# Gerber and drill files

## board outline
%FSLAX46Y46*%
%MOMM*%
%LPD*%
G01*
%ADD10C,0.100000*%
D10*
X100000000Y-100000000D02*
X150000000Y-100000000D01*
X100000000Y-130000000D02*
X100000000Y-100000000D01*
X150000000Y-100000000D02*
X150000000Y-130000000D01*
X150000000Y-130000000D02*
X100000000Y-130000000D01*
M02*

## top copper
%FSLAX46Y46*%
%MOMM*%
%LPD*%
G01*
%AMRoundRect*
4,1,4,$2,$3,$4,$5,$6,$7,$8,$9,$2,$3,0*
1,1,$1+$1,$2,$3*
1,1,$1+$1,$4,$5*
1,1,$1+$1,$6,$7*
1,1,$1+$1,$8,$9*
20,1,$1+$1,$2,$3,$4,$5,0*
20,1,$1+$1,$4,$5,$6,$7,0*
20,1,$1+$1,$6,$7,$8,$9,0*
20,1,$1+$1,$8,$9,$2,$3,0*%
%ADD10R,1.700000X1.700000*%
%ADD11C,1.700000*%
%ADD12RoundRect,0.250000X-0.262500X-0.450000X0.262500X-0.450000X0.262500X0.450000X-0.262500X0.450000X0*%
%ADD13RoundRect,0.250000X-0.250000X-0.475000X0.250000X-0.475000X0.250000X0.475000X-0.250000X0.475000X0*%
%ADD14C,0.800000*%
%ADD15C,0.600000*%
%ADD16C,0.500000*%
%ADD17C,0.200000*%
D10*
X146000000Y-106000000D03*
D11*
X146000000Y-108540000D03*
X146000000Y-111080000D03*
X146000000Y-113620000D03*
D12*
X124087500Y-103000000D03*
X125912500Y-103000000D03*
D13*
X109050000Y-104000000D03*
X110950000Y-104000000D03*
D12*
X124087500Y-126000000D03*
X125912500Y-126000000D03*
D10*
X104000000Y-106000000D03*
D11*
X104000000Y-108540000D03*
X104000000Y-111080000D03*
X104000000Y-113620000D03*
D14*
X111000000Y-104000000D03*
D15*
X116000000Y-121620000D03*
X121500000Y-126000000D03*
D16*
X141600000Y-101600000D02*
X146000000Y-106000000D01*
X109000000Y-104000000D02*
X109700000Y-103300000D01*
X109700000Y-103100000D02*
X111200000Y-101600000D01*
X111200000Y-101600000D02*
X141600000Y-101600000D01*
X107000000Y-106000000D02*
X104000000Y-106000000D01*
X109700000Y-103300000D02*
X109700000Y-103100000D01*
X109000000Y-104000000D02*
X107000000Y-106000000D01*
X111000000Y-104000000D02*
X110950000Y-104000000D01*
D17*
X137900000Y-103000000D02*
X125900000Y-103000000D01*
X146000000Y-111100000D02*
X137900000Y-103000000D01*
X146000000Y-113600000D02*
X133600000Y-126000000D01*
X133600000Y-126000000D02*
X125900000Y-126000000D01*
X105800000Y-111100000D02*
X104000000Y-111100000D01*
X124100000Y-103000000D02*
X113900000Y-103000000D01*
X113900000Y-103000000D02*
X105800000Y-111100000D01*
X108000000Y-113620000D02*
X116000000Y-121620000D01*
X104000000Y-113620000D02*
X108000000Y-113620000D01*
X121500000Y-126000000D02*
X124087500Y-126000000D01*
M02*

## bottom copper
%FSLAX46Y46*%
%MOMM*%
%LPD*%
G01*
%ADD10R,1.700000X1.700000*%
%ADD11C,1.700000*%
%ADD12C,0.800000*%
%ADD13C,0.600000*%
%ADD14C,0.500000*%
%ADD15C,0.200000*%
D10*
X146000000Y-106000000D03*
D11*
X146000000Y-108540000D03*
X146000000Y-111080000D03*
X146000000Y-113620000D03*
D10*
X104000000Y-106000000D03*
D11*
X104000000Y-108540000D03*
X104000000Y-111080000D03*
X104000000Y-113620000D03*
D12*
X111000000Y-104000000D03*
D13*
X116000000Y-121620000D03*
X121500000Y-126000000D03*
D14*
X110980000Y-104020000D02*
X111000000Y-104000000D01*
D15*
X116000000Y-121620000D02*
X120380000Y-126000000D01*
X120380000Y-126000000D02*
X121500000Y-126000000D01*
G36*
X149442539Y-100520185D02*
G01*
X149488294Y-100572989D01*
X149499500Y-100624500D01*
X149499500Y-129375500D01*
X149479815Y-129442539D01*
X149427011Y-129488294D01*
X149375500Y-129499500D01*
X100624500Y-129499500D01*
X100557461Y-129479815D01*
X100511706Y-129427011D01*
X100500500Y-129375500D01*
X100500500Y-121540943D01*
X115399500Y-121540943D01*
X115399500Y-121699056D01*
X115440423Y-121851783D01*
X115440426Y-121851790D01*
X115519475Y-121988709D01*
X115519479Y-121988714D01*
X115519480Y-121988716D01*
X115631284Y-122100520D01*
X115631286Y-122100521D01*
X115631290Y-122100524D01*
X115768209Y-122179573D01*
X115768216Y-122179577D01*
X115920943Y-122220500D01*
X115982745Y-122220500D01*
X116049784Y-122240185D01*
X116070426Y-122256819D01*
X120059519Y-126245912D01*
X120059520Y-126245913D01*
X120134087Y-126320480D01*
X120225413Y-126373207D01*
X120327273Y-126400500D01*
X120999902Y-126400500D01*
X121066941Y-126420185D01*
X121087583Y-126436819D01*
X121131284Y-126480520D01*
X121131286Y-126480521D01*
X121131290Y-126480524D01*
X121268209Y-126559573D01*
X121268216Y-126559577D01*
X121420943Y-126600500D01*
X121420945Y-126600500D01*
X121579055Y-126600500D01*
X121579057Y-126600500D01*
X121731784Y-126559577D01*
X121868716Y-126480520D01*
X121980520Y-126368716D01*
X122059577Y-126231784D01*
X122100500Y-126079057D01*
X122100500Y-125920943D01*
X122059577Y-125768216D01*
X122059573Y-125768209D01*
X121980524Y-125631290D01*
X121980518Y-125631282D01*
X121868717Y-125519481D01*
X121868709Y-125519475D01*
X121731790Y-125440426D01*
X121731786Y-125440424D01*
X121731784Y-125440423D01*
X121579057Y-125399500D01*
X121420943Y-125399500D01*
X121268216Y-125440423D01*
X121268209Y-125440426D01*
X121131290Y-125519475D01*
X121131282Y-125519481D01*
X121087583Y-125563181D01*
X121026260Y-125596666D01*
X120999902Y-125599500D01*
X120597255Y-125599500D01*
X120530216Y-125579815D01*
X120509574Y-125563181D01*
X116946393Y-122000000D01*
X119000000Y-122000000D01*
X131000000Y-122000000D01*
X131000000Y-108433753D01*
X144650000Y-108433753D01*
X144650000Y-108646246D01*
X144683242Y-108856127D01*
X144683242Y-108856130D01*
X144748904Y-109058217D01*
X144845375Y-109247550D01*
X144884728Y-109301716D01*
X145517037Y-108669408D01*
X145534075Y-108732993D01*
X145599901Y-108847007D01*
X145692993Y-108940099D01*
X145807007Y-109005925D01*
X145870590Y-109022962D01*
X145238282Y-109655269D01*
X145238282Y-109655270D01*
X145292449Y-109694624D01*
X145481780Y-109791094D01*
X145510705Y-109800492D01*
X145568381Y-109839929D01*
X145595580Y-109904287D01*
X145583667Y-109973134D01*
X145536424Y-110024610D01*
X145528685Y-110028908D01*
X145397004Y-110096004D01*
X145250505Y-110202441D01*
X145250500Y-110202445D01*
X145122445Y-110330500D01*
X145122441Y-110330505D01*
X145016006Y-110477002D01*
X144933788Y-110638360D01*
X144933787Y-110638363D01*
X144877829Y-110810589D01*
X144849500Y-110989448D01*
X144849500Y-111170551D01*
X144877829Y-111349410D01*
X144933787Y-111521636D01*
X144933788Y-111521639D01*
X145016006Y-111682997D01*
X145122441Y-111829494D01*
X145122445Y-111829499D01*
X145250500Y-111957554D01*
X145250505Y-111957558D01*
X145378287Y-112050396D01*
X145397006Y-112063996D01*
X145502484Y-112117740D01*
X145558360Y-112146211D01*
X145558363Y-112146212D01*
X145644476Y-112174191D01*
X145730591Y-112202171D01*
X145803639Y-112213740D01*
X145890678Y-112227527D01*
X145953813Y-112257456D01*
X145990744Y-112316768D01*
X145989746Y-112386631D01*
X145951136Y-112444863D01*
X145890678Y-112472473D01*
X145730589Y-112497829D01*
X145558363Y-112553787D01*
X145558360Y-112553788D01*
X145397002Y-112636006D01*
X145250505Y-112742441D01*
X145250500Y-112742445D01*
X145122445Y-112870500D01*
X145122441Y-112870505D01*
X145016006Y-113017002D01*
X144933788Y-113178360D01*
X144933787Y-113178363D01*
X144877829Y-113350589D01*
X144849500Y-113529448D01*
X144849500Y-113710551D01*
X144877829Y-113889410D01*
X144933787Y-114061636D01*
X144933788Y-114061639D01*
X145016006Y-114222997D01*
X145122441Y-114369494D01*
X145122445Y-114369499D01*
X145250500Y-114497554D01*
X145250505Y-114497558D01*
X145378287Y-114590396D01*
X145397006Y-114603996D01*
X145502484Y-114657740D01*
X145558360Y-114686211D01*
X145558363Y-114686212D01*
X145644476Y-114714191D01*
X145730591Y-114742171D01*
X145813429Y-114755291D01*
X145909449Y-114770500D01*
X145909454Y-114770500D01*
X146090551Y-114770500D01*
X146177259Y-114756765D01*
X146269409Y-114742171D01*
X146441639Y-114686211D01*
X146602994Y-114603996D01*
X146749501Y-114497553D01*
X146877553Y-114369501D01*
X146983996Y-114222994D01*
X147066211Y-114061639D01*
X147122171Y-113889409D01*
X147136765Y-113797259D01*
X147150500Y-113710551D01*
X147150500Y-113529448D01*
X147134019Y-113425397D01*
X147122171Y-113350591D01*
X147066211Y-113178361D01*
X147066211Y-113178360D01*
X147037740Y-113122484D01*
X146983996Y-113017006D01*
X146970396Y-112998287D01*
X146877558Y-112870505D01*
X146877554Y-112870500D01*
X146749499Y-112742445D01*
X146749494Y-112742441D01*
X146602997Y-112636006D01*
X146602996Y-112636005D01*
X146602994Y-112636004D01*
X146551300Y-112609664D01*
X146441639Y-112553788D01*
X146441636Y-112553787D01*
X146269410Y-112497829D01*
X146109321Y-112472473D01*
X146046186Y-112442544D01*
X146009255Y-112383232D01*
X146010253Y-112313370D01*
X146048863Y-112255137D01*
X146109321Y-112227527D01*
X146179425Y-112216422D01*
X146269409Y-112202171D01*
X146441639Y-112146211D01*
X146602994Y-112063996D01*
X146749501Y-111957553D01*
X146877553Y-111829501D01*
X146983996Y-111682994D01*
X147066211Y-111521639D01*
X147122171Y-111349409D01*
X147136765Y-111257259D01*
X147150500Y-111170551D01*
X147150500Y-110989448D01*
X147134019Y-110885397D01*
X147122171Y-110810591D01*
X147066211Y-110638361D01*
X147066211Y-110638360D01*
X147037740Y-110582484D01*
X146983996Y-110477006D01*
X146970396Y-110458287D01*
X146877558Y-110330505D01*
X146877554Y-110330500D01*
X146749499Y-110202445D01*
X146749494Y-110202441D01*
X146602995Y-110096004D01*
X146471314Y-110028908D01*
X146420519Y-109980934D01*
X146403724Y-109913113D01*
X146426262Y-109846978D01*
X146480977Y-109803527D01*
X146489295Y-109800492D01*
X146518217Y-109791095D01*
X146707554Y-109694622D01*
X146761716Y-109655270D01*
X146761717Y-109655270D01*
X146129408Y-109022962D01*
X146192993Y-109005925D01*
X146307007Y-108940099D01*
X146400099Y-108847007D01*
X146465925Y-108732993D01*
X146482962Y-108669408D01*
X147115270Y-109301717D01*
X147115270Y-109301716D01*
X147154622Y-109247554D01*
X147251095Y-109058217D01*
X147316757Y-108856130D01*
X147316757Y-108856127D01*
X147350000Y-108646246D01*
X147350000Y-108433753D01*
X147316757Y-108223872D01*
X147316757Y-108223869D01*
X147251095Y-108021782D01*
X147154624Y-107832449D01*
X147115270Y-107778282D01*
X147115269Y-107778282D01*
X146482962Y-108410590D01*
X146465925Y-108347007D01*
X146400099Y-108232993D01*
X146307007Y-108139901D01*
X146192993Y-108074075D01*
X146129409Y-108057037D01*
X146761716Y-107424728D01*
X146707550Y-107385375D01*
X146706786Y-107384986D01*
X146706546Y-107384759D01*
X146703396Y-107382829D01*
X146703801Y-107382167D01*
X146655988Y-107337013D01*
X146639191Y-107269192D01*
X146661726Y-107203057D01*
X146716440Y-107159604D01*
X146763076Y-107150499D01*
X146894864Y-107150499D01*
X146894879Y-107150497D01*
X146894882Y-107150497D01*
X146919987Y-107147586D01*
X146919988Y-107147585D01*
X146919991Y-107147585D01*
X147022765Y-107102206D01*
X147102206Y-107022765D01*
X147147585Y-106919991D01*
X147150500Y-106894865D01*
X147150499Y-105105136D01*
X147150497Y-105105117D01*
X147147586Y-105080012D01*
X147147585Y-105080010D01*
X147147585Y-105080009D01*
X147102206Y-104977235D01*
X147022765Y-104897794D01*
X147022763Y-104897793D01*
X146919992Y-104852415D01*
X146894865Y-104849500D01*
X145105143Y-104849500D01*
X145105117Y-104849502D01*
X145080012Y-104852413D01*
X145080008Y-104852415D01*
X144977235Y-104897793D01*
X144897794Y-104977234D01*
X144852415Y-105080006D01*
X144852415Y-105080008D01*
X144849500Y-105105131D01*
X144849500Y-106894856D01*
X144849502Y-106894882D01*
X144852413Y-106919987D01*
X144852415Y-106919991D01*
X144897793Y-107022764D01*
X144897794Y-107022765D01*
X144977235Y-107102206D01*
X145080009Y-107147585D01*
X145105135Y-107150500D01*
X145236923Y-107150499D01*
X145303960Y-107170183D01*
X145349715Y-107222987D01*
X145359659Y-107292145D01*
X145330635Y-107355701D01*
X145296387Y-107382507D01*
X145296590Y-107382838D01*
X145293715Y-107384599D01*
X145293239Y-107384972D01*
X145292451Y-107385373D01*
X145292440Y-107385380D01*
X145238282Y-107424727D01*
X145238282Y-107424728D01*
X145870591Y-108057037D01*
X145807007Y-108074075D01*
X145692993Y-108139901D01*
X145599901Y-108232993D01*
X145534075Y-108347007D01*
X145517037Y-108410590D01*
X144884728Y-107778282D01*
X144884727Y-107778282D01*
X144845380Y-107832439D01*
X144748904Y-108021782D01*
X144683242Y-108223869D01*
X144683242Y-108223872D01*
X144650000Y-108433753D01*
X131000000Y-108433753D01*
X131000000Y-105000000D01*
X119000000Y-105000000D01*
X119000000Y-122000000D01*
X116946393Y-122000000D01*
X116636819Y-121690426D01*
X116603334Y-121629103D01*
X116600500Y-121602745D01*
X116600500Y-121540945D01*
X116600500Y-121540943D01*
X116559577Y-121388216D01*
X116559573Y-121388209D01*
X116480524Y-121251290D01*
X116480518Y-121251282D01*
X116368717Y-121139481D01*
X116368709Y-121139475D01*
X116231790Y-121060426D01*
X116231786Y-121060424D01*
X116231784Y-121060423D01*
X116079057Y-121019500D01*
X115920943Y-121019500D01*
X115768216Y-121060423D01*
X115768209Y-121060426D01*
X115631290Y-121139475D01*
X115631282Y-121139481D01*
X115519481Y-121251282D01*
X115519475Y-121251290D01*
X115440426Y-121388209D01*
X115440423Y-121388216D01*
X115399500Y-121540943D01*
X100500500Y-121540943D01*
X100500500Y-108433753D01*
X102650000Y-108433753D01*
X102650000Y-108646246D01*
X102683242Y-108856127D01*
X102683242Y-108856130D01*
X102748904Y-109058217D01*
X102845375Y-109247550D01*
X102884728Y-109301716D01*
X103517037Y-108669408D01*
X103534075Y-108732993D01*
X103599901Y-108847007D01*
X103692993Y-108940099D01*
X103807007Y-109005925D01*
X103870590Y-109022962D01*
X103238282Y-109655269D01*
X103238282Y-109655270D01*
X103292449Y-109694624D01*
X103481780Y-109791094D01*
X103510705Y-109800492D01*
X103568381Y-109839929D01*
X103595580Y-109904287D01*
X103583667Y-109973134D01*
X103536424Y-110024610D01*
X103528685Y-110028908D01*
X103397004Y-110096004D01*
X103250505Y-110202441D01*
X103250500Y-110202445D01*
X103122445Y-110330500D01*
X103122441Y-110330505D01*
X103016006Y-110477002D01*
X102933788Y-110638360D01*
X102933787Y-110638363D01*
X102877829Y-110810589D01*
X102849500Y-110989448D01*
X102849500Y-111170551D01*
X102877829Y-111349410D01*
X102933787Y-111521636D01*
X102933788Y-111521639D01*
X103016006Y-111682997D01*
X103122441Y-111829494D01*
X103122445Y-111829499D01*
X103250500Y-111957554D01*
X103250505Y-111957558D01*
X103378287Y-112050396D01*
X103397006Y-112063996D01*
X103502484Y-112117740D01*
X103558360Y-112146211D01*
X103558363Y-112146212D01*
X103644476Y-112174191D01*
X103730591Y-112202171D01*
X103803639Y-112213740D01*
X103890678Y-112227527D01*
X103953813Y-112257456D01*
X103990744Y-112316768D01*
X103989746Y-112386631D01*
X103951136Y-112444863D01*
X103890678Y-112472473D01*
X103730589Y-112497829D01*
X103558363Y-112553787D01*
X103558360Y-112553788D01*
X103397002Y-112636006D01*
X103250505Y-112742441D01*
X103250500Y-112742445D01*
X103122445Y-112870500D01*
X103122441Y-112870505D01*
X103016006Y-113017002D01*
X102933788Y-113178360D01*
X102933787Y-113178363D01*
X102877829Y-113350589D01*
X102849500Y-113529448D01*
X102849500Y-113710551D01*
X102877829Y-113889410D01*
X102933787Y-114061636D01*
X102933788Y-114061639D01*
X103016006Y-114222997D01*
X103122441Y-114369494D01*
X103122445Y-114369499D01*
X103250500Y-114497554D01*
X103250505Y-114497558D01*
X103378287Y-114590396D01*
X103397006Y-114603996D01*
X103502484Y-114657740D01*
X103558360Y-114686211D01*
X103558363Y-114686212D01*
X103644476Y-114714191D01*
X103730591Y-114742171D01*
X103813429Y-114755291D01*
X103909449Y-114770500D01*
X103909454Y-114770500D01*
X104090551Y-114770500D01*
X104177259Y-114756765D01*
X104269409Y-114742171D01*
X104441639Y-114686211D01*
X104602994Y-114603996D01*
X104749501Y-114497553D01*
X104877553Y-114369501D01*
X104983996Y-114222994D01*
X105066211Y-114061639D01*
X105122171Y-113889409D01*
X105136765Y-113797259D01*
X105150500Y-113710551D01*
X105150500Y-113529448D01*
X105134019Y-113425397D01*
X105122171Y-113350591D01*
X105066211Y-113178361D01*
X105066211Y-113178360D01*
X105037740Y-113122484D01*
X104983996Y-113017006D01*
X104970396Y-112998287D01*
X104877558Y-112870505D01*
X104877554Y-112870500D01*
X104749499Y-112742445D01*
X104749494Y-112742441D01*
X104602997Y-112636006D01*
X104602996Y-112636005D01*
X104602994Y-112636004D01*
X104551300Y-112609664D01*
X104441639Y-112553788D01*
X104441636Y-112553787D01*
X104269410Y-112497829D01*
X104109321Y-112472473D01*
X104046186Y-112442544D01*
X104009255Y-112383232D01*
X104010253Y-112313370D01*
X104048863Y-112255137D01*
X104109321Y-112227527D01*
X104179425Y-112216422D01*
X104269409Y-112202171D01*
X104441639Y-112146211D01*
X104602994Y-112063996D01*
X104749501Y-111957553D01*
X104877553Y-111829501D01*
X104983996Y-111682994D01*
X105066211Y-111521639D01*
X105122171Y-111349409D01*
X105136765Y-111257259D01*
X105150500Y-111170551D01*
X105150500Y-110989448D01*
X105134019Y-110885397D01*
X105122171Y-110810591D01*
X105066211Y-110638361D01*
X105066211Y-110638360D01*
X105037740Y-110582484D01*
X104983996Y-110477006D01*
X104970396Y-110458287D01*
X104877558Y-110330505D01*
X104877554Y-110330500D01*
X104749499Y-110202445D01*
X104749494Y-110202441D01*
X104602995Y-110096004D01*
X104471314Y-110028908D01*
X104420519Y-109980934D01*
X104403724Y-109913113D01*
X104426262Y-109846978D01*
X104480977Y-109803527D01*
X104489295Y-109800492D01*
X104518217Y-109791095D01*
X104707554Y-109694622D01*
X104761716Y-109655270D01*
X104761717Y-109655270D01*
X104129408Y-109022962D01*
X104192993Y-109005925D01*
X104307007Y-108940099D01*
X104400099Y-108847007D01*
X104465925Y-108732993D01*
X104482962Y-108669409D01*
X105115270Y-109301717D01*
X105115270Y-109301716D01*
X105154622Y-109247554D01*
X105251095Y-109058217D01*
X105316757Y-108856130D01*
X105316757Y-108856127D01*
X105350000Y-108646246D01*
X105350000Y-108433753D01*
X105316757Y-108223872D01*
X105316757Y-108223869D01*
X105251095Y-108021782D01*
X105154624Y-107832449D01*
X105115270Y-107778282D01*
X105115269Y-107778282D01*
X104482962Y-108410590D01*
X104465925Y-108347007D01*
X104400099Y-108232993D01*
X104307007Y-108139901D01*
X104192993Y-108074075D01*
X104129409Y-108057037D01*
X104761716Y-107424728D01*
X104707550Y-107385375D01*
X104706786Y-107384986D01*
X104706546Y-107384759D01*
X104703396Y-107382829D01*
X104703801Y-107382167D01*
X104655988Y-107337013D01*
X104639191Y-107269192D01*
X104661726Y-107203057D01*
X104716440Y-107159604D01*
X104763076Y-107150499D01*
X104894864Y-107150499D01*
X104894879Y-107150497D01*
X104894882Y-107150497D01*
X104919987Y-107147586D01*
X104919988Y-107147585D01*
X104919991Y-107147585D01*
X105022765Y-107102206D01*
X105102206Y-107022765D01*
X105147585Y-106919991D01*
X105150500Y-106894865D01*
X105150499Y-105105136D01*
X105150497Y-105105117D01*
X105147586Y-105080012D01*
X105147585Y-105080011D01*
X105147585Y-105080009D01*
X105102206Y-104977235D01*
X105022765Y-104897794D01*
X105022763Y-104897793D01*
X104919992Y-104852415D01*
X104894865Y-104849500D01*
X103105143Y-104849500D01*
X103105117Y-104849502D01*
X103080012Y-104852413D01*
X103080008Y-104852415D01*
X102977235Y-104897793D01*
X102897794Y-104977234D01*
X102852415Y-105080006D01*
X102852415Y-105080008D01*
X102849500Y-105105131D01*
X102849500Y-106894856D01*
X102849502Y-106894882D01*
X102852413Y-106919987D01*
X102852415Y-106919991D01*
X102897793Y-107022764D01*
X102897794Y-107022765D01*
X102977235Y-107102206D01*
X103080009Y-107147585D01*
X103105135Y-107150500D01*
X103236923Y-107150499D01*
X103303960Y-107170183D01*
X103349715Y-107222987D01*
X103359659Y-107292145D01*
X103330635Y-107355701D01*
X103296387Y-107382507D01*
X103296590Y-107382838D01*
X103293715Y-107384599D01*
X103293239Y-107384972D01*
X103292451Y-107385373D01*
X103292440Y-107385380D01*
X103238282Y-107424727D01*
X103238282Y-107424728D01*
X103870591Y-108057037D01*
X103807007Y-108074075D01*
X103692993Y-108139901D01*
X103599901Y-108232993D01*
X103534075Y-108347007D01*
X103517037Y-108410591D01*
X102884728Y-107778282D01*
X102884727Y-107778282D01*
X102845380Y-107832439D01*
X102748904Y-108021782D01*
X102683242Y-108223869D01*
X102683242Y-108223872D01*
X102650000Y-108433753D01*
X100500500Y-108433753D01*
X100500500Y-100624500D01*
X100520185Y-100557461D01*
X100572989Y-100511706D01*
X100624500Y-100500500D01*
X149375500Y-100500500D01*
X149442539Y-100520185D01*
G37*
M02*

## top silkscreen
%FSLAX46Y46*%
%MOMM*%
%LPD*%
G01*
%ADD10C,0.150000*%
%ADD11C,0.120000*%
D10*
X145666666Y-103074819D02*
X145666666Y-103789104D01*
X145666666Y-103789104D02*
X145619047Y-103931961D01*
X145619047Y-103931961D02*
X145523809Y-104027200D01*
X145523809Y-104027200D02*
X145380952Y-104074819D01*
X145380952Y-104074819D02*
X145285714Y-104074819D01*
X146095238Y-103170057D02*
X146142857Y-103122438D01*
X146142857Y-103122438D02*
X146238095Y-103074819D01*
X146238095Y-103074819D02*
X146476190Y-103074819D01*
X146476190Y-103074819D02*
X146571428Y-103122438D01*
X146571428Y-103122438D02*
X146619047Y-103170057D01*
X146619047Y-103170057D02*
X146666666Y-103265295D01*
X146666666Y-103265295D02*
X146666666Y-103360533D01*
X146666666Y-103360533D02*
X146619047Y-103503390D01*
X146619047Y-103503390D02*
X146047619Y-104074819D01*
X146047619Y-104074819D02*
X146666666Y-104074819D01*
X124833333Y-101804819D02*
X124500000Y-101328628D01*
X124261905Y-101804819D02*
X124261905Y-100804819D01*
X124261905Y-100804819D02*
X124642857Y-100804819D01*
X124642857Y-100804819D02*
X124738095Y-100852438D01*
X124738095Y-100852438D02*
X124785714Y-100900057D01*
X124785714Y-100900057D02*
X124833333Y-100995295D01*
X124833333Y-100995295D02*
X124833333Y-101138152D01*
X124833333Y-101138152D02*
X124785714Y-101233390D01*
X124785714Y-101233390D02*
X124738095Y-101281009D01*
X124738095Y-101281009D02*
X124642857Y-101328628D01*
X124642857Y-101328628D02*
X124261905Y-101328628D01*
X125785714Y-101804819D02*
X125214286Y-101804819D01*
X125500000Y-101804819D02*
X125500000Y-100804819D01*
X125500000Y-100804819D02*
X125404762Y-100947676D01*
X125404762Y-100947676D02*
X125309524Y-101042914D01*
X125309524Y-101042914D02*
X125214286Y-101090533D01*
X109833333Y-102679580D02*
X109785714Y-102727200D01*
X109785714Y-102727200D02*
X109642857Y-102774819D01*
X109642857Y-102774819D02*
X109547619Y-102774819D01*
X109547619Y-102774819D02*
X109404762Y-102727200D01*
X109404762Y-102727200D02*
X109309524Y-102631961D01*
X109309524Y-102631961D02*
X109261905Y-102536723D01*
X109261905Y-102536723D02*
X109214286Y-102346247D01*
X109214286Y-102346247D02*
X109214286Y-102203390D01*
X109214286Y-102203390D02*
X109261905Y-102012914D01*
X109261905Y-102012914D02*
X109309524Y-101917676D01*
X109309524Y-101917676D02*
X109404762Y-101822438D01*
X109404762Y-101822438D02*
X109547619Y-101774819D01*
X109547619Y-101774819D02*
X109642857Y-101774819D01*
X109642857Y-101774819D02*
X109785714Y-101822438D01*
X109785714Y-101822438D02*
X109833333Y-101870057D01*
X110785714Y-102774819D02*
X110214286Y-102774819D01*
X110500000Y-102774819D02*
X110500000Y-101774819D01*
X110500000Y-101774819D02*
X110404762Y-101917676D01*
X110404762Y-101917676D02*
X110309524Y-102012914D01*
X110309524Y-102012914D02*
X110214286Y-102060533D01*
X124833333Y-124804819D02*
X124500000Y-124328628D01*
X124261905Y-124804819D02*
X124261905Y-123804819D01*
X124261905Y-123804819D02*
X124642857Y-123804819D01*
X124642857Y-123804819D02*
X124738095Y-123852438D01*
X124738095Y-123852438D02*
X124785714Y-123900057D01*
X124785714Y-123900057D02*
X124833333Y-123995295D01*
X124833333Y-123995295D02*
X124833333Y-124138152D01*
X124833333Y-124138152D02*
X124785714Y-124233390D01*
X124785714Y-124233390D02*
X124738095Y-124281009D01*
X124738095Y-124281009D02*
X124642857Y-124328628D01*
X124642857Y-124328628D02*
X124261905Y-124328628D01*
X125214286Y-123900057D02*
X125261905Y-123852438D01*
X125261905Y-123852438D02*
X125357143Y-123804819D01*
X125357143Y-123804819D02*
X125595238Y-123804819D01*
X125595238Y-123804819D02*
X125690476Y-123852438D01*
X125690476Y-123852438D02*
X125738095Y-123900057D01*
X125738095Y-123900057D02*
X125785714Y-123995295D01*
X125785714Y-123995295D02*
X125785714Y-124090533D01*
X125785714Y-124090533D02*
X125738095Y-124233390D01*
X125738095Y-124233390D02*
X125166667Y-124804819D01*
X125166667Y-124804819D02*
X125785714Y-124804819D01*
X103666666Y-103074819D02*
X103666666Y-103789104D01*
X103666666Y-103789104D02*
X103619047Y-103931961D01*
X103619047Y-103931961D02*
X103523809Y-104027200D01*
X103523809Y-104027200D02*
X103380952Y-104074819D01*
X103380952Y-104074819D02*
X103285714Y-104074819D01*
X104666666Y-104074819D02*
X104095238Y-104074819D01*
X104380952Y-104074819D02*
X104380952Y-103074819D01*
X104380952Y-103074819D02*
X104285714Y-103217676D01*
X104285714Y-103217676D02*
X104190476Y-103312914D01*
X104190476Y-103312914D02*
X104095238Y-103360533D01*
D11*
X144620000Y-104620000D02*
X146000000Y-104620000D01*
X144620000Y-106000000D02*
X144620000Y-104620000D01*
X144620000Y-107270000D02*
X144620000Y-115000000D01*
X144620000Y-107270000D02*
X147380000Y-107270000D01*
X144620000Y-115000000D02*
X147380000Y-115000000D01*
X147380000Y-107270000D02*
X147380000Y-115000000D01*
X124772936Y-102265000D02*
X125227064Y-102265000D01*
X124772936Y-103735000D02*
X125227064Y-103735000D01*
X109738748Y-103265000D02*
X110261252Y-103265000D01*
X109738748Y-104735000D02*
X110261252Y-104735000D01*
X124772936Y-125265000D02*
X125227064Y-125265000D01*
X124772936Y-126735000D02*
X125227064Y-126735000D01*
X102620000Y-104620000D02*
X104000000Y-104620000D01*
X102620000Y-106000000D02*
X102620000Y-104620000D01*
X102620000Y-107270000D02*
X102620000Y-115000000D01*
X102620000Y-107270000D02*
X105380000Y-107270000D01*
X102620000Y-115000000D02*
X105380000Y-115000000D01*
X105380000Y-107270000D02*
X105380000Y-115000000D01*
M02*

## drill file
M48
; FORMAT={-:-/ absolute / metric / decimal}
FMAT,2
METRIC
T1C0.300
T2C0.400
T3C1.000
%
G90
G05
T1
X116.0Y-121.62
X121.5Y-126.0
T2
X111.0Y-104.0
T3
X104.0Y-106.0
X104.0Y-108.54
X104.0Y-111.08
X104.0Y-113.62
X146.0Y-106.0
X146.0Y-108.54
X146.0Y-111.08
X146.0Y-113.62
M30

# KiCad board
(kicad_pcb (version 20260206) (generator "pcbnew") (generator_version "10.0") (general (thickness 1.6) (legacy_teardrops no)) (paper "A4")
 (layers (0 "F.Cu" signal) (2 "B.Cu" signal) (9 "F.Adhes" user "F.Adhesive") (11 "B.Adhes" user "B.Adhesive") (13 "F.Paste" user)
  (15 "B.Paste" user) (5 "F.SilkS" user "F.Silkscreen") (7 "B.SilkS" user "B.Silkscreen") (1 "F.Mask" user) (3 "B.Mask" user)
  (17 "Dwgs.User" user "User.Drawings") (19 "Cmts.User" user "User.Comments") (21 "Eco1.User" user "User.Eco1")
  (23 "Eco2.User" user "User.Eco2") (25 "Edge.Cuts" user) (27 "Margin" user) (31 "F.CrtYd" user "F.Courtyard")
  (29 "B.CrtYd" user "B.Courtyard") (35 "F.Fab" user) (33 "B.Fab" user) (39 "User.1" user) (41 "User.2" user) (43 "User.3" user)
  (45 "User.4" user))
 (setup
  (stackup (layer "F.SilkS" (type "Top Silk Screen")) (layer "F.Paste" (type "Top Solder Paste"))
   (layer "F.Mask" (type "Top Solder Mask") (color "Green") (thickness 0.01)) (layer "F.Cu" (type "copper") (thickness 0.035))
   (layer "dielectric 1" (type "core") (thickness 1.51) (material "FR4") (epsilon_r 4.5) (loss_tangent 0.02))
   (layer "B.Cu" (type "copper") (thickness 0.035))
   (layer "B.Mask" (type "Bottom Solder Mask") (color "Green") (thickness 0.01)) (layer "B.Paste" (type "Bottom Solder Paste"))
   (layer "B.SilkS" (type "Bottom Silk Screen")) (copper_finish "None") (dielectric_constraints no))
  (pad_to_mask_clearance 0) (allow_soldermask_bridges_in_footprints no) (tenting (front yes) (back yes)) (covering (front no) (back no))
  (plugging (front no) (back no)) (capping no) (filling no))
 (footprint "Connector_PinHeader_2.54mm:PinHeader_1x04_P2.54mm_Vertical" (layer "F.Cu") (at 146 106)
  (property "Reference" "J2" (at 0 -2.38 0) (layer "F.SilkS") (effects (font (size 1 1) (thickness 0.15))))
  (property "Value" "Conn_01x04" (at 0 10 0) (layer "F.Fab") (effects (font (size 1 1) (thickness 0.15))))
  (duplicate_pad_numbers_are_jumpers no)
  (fp_line (start -1.38 -1.38) (end 0 -1.38) (stroke (width 0.12) (type solid)) (layer "F.SilkS"))
  (fp_line (start -1.38 0) (end -1.38 -1.38) (stroke (width 0.12) (type solid)) (layer "F.SilkS"))
  (fp_line (start -1.38 1.27) (end -1.38 9) (stroke (width 0.12) (type solid)) (layer "F.SilkS"))
  (fp_line (start -1.38 1.27) (end 1.38 1.27) (stroke (width 0.12) (type solid)) (layer "F.SilkS"))
  (fp_line (start -1.38 9) (end 1.38 9) (stroke (width 0.12) (type solid)) (layer "F.SilkS"))
  (fp_line (start 1.38 1.27) (end 1.38 9) (stroke (width 0.12) (type solid)) (layer "F.SilkS"))
  (pad "1" thru_hole rect (at 0 0) (size 1.7 1.7) (drill 1) (layers "*.Cu" "*.Mask") (remove_unused_layers no) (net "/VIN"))
  (pad "2" thru_hole circle (at 0 2.54) (size 1.7 1.7) (drill 1) (layers "*.Cu" "*.Mask") (remove_unused_layers no) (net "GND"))
  (pad "3" thru_hole circle (at 0 5.08) (size 1.7 1.7) (drill 1) (layers "*.Cu" "*.Mask") (remove_unused_layers no) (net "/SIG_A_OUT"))
  (pad "4" thru_hole circle (at 0 7.62) (size 1.7 1.7) (drill 1) (layers "*.Cu" "*.Mask") (remove_unused_layers no) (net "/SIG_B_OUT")))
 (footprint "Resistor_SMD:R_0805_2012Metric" (layer "F.Cu") (at 125 103)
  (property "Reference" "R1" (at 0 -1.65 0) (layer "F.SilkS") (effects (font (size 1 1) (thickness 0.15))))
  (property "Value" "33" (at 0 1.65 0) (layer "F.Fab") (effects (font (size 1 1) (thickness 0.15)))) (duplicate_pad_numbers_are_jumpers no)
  (fp_line (start -0.227064 -0.735) (end 0.227064 -0.735) (stroke (width 0.12) (type solid)) (layer "F.SilkS"))
  (fp_line (start -0.227064 0.735) (end 0.227064 0.735) (stroke (width 0.12) (type solid)) (layer "F.SilkS"))
  (pad "1" smd roundrect (at -0.9125 0) (size 1.025 1.4) (layers "F.Cu" "F.Mask" "F.Paste") (roundrect_rratio 0.243902) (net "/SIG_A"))
  (pad "2" smd roundrect (at 0.9125 0) (size 1.025 1.4) (layers "F.Cu" "F.Mask" "F.Paste") (roundrect_rratio 0.243902) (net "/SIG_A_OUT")))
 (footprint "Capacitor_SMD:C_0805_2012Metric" (layer "F.Cu") (at 110 104)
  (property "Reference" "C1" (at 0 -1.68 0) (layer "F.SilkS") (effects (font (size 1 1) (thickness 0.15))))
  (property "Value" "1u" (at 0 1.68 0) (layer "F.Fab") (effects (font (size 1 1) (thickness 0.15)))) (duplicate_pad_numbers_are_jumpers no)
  (fp_line (start -0.261252 -0.735) (end 0.261252 -0.735) (stroke (width 0.12) (type solid)) (layer "F.SilkS"))
  (fp_line (start -0.261252 0.735) (end 0.261252 0.735) (stroke (width 0.12) (type solid)) (layer "F.SilkS"))
  (pad "1" smd roundrect (at -0.95 0) (size 1 1.45) (layers "F.Cu" "F.Mask" "F.Paste") (roundrect_rratio 0.25) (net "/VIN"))
  (pad "2" smd roundrect (at 0.95 0) (size 1 1.45) (layers "F.Cu" "F.Mask" "F.Paste") (roundrect_rratio 0.25) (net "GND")))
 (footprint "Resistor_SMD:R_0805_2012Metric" (layer "F.Cu") (at 125 126)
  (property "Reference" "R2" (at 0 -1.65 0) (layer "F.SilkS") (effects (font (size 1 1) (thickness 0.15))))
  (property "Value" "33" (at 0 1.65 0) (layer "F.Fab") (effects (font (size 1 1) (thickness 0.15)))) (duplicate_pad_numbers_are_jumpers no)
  (fp_line (start -0.227064 -0.735) (end 0.227064 -0.735) (stroke (width 0.12) (type solid)) (layer "F.SilkS"))
  (fp_line (start -0.227064 0.735) (end 0.227064 0.735) (stroke (width 0.12) (type solid)) (layer "F.SilkS"))
  (pad "1" smd roundrect (at -0.9125 0) (size 1.025 1.4) (layers "F.Cu" "F.Mask" "F.Paste") (roundrect_rratio 0.243902) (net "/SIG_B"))
  (pad "2" smd roundrect (at 0.9125 0) (size 1.025 1.4) (layers "F.Cu" "F.Mask" "F.Paste") (roundrect_rratio 0.243902) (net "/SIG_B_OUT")))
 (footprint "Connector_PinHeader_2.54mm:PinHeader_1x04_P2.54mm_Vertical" (layer "F.Cu") (at 104 106)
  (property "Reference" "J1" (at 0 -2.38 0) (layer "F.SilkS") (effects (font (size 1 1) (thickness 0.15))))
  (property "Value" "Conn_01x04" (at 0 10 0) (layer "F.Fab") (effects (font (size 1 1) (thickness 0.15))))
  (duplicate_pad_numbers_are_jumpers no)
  (fp_line (start -1.38 -1.38) (end 0 -1.38) (stroke (width 0.12) (type solid)) (layer "F.SilkS"))
  (fp_line (start -1.38 0) (end -1.38 -1.38) (stroke (width 0.12) (type solid)) (layer "F.SilkS"))
  (fp_line (start -1.38 1.27) (end -1.38 9) (stroke (width 0.12) (type solid)) (layer "F.SilkS"))
  (fp_line (start -1.38 1.27) (end 1.38 1.27) (stroke (width 0.12) (type solid)) (layer "F.SilkS"))
  (fp_line (start -1.38 9) (end 1.38 9) (stroke (width 0.12) (type solid)) (layer "F.SilkS"))
  (fp_line (start 1.38 1.27) (end 1.38 9) (stroke (width 0.12) (type solid)) (layer "F.SilkS"))
  (pad "1" thru_hole rect (at 0 0) (size 1.7 1.7) (drill 1) (layers "*.Cu" "*.Mask") (remove_unused_layers no) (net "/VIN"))
  (pad "2" thru_hole circle (at 0 2.54) (size 1.7 1.7) (drill 1) (layers "*.Cu" "*.Mask") (remove_unused_layers no) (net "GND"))
  (pad "3" thru_hole circle (at 0 5.08) (size 1.7 1.7) (drill 1) (layers "*.Cu" "*.Mask") (remove_unused_layers no) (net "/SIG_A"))
  (pad "4" thru_hole circle (at 0 7.62) (size 1.7 1.7) (drill 1) (layers "*.Cu" "*.Mask") (remove_unused_layers no) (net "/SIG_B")))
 (gr_line (start 100 100) (end 150 100) (stroke (width 0.1) (type default)) (layer "Edge.Cuts"))
 (gr_line (start 100 130) (end 100 100) (stroke (width 0.1) (type default)) (layer "Edge.Cuts"))
 (gr_line (start 150 100) (end 150 130) (stroke (width 0.1) (type default)) (layer "Edge.Cuts"))
 (gr_line (start 150 130) (end 100 130) (stroke (width 0.1) (type default)) (layer "Edge.Cuts"))
 (segment (start 141.6 101.6) (end 146 106) (width 0.5) (layer "F.Cu") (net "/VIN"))
 (segment (start 109 104) (end 109.7 103.3) (width 0.5) (layer "F.Cu") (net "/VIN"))
 (segment (start 109.7 103.1) (end 111.2 101.6) (width 0.5) (layer "F.Cu") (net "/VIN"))
 (segment (start 111.2 101.6) (end 141.6 101.6) (width 0.5) (layer "F.Cu") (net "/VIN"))
 (segment (start 107 106) (end 104 106) (width 0.5) (layer "F.Cu") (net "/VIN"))
 (segment (start 109.7 103.3) (end 109.7 103.1) (width 0.5) (layer "F.Cu") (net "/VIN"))
 (segment (start 109 104) (end 107 106) (width 0.5) (layer "F.Cu") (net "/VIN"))
 (segment (start 111 104) (end 110.95 104) (width 0.5) (layer "F.Cu") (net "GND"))
 (via (at 111 104) (size 0.8) (drill 0.4) (layers "F.Cu" "B.Cu") (capping yes) (filling yes) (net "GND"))
 (segment (start 110.98 104.02) (end 111 104) (width 0.5) (layer "B.Cu") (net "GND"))
 (segment (start 137.9 103) (end 125.9 103) (width 0.2) (layer "F.Cu") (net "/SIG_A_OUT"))
 (segment (start 146 111.1) (end 137.9 103) (width 0.2) (layer "F.Cu") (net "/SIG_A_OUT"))
 (segment (start 146 113.6) (end 133.6 126) (width 0.2) (layer "F.Cu") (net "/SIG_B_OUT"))
 (segment (start 133.6 126) (end 125.9 126) (width 0.2) (layer "F.Cu") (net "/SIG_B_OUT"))
 (segment (start 105.8 111.1) (end 104 111.1) (width 0.2) (layer "F.Cu") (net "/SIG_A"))
 (segment (start 124.1 103) (end 113.9 103) (width 0.2) (layer "F.Cu") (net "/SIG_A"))
 (segment (start 113.9 103) (end 105.8 111.1) (width 0.2) (layer "F.Cu") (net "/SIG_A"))
 (segment (start 108 113.62) (end 116 121.62) (width 0.2) (locked yes) (layer "F.Cu") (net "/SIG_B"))
 (segment (start 104 113.62) (end 108 113.62) (width 0.2) (locked yes) (layer "F.Cu") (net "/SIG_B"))
 (segment (start 121.5 126) (end 124.0875 126) (width 0.2) (locked yes) (layer "F.Cu") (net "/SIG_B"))
 (via (at 116 121.62) (size 0.6) (drill 0.3) (layers "F.Cu" "B.Cu") (locked yes) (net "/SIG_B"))
 (via (at 121.5 126) (size 0.6) (drill 0.3) (layers "F.Cu" "B.Cu") (locked yes) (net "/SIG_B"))
 (segment (start 116 121.62) (end 120.38 126) (width 0.2) (locked yes) (layer "B.Cu") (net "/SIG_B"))
 (segment (start 120.38 126) (end 121.5 126) (width 0.2) (locked yes) (layer "B.Cu") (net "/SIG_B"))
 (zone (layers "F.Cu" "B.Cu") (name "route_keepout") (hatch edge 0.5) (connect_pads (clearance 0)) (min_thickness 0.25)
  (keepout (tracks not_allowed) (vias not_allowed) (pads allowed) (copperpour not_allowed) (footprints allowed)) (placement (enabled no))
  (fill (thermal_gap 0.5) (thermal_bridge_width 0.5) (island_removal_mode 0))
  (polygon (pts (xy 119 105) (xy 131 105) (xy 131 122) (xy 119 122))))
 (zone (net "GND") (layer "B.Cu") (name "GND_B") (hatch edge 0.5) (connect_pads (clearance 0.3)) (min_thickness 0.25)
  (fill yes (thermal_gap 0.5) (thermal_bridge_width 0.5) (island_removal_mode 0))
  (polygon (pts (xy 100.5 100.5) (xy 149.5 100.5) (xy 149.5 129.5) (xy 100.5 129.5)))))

